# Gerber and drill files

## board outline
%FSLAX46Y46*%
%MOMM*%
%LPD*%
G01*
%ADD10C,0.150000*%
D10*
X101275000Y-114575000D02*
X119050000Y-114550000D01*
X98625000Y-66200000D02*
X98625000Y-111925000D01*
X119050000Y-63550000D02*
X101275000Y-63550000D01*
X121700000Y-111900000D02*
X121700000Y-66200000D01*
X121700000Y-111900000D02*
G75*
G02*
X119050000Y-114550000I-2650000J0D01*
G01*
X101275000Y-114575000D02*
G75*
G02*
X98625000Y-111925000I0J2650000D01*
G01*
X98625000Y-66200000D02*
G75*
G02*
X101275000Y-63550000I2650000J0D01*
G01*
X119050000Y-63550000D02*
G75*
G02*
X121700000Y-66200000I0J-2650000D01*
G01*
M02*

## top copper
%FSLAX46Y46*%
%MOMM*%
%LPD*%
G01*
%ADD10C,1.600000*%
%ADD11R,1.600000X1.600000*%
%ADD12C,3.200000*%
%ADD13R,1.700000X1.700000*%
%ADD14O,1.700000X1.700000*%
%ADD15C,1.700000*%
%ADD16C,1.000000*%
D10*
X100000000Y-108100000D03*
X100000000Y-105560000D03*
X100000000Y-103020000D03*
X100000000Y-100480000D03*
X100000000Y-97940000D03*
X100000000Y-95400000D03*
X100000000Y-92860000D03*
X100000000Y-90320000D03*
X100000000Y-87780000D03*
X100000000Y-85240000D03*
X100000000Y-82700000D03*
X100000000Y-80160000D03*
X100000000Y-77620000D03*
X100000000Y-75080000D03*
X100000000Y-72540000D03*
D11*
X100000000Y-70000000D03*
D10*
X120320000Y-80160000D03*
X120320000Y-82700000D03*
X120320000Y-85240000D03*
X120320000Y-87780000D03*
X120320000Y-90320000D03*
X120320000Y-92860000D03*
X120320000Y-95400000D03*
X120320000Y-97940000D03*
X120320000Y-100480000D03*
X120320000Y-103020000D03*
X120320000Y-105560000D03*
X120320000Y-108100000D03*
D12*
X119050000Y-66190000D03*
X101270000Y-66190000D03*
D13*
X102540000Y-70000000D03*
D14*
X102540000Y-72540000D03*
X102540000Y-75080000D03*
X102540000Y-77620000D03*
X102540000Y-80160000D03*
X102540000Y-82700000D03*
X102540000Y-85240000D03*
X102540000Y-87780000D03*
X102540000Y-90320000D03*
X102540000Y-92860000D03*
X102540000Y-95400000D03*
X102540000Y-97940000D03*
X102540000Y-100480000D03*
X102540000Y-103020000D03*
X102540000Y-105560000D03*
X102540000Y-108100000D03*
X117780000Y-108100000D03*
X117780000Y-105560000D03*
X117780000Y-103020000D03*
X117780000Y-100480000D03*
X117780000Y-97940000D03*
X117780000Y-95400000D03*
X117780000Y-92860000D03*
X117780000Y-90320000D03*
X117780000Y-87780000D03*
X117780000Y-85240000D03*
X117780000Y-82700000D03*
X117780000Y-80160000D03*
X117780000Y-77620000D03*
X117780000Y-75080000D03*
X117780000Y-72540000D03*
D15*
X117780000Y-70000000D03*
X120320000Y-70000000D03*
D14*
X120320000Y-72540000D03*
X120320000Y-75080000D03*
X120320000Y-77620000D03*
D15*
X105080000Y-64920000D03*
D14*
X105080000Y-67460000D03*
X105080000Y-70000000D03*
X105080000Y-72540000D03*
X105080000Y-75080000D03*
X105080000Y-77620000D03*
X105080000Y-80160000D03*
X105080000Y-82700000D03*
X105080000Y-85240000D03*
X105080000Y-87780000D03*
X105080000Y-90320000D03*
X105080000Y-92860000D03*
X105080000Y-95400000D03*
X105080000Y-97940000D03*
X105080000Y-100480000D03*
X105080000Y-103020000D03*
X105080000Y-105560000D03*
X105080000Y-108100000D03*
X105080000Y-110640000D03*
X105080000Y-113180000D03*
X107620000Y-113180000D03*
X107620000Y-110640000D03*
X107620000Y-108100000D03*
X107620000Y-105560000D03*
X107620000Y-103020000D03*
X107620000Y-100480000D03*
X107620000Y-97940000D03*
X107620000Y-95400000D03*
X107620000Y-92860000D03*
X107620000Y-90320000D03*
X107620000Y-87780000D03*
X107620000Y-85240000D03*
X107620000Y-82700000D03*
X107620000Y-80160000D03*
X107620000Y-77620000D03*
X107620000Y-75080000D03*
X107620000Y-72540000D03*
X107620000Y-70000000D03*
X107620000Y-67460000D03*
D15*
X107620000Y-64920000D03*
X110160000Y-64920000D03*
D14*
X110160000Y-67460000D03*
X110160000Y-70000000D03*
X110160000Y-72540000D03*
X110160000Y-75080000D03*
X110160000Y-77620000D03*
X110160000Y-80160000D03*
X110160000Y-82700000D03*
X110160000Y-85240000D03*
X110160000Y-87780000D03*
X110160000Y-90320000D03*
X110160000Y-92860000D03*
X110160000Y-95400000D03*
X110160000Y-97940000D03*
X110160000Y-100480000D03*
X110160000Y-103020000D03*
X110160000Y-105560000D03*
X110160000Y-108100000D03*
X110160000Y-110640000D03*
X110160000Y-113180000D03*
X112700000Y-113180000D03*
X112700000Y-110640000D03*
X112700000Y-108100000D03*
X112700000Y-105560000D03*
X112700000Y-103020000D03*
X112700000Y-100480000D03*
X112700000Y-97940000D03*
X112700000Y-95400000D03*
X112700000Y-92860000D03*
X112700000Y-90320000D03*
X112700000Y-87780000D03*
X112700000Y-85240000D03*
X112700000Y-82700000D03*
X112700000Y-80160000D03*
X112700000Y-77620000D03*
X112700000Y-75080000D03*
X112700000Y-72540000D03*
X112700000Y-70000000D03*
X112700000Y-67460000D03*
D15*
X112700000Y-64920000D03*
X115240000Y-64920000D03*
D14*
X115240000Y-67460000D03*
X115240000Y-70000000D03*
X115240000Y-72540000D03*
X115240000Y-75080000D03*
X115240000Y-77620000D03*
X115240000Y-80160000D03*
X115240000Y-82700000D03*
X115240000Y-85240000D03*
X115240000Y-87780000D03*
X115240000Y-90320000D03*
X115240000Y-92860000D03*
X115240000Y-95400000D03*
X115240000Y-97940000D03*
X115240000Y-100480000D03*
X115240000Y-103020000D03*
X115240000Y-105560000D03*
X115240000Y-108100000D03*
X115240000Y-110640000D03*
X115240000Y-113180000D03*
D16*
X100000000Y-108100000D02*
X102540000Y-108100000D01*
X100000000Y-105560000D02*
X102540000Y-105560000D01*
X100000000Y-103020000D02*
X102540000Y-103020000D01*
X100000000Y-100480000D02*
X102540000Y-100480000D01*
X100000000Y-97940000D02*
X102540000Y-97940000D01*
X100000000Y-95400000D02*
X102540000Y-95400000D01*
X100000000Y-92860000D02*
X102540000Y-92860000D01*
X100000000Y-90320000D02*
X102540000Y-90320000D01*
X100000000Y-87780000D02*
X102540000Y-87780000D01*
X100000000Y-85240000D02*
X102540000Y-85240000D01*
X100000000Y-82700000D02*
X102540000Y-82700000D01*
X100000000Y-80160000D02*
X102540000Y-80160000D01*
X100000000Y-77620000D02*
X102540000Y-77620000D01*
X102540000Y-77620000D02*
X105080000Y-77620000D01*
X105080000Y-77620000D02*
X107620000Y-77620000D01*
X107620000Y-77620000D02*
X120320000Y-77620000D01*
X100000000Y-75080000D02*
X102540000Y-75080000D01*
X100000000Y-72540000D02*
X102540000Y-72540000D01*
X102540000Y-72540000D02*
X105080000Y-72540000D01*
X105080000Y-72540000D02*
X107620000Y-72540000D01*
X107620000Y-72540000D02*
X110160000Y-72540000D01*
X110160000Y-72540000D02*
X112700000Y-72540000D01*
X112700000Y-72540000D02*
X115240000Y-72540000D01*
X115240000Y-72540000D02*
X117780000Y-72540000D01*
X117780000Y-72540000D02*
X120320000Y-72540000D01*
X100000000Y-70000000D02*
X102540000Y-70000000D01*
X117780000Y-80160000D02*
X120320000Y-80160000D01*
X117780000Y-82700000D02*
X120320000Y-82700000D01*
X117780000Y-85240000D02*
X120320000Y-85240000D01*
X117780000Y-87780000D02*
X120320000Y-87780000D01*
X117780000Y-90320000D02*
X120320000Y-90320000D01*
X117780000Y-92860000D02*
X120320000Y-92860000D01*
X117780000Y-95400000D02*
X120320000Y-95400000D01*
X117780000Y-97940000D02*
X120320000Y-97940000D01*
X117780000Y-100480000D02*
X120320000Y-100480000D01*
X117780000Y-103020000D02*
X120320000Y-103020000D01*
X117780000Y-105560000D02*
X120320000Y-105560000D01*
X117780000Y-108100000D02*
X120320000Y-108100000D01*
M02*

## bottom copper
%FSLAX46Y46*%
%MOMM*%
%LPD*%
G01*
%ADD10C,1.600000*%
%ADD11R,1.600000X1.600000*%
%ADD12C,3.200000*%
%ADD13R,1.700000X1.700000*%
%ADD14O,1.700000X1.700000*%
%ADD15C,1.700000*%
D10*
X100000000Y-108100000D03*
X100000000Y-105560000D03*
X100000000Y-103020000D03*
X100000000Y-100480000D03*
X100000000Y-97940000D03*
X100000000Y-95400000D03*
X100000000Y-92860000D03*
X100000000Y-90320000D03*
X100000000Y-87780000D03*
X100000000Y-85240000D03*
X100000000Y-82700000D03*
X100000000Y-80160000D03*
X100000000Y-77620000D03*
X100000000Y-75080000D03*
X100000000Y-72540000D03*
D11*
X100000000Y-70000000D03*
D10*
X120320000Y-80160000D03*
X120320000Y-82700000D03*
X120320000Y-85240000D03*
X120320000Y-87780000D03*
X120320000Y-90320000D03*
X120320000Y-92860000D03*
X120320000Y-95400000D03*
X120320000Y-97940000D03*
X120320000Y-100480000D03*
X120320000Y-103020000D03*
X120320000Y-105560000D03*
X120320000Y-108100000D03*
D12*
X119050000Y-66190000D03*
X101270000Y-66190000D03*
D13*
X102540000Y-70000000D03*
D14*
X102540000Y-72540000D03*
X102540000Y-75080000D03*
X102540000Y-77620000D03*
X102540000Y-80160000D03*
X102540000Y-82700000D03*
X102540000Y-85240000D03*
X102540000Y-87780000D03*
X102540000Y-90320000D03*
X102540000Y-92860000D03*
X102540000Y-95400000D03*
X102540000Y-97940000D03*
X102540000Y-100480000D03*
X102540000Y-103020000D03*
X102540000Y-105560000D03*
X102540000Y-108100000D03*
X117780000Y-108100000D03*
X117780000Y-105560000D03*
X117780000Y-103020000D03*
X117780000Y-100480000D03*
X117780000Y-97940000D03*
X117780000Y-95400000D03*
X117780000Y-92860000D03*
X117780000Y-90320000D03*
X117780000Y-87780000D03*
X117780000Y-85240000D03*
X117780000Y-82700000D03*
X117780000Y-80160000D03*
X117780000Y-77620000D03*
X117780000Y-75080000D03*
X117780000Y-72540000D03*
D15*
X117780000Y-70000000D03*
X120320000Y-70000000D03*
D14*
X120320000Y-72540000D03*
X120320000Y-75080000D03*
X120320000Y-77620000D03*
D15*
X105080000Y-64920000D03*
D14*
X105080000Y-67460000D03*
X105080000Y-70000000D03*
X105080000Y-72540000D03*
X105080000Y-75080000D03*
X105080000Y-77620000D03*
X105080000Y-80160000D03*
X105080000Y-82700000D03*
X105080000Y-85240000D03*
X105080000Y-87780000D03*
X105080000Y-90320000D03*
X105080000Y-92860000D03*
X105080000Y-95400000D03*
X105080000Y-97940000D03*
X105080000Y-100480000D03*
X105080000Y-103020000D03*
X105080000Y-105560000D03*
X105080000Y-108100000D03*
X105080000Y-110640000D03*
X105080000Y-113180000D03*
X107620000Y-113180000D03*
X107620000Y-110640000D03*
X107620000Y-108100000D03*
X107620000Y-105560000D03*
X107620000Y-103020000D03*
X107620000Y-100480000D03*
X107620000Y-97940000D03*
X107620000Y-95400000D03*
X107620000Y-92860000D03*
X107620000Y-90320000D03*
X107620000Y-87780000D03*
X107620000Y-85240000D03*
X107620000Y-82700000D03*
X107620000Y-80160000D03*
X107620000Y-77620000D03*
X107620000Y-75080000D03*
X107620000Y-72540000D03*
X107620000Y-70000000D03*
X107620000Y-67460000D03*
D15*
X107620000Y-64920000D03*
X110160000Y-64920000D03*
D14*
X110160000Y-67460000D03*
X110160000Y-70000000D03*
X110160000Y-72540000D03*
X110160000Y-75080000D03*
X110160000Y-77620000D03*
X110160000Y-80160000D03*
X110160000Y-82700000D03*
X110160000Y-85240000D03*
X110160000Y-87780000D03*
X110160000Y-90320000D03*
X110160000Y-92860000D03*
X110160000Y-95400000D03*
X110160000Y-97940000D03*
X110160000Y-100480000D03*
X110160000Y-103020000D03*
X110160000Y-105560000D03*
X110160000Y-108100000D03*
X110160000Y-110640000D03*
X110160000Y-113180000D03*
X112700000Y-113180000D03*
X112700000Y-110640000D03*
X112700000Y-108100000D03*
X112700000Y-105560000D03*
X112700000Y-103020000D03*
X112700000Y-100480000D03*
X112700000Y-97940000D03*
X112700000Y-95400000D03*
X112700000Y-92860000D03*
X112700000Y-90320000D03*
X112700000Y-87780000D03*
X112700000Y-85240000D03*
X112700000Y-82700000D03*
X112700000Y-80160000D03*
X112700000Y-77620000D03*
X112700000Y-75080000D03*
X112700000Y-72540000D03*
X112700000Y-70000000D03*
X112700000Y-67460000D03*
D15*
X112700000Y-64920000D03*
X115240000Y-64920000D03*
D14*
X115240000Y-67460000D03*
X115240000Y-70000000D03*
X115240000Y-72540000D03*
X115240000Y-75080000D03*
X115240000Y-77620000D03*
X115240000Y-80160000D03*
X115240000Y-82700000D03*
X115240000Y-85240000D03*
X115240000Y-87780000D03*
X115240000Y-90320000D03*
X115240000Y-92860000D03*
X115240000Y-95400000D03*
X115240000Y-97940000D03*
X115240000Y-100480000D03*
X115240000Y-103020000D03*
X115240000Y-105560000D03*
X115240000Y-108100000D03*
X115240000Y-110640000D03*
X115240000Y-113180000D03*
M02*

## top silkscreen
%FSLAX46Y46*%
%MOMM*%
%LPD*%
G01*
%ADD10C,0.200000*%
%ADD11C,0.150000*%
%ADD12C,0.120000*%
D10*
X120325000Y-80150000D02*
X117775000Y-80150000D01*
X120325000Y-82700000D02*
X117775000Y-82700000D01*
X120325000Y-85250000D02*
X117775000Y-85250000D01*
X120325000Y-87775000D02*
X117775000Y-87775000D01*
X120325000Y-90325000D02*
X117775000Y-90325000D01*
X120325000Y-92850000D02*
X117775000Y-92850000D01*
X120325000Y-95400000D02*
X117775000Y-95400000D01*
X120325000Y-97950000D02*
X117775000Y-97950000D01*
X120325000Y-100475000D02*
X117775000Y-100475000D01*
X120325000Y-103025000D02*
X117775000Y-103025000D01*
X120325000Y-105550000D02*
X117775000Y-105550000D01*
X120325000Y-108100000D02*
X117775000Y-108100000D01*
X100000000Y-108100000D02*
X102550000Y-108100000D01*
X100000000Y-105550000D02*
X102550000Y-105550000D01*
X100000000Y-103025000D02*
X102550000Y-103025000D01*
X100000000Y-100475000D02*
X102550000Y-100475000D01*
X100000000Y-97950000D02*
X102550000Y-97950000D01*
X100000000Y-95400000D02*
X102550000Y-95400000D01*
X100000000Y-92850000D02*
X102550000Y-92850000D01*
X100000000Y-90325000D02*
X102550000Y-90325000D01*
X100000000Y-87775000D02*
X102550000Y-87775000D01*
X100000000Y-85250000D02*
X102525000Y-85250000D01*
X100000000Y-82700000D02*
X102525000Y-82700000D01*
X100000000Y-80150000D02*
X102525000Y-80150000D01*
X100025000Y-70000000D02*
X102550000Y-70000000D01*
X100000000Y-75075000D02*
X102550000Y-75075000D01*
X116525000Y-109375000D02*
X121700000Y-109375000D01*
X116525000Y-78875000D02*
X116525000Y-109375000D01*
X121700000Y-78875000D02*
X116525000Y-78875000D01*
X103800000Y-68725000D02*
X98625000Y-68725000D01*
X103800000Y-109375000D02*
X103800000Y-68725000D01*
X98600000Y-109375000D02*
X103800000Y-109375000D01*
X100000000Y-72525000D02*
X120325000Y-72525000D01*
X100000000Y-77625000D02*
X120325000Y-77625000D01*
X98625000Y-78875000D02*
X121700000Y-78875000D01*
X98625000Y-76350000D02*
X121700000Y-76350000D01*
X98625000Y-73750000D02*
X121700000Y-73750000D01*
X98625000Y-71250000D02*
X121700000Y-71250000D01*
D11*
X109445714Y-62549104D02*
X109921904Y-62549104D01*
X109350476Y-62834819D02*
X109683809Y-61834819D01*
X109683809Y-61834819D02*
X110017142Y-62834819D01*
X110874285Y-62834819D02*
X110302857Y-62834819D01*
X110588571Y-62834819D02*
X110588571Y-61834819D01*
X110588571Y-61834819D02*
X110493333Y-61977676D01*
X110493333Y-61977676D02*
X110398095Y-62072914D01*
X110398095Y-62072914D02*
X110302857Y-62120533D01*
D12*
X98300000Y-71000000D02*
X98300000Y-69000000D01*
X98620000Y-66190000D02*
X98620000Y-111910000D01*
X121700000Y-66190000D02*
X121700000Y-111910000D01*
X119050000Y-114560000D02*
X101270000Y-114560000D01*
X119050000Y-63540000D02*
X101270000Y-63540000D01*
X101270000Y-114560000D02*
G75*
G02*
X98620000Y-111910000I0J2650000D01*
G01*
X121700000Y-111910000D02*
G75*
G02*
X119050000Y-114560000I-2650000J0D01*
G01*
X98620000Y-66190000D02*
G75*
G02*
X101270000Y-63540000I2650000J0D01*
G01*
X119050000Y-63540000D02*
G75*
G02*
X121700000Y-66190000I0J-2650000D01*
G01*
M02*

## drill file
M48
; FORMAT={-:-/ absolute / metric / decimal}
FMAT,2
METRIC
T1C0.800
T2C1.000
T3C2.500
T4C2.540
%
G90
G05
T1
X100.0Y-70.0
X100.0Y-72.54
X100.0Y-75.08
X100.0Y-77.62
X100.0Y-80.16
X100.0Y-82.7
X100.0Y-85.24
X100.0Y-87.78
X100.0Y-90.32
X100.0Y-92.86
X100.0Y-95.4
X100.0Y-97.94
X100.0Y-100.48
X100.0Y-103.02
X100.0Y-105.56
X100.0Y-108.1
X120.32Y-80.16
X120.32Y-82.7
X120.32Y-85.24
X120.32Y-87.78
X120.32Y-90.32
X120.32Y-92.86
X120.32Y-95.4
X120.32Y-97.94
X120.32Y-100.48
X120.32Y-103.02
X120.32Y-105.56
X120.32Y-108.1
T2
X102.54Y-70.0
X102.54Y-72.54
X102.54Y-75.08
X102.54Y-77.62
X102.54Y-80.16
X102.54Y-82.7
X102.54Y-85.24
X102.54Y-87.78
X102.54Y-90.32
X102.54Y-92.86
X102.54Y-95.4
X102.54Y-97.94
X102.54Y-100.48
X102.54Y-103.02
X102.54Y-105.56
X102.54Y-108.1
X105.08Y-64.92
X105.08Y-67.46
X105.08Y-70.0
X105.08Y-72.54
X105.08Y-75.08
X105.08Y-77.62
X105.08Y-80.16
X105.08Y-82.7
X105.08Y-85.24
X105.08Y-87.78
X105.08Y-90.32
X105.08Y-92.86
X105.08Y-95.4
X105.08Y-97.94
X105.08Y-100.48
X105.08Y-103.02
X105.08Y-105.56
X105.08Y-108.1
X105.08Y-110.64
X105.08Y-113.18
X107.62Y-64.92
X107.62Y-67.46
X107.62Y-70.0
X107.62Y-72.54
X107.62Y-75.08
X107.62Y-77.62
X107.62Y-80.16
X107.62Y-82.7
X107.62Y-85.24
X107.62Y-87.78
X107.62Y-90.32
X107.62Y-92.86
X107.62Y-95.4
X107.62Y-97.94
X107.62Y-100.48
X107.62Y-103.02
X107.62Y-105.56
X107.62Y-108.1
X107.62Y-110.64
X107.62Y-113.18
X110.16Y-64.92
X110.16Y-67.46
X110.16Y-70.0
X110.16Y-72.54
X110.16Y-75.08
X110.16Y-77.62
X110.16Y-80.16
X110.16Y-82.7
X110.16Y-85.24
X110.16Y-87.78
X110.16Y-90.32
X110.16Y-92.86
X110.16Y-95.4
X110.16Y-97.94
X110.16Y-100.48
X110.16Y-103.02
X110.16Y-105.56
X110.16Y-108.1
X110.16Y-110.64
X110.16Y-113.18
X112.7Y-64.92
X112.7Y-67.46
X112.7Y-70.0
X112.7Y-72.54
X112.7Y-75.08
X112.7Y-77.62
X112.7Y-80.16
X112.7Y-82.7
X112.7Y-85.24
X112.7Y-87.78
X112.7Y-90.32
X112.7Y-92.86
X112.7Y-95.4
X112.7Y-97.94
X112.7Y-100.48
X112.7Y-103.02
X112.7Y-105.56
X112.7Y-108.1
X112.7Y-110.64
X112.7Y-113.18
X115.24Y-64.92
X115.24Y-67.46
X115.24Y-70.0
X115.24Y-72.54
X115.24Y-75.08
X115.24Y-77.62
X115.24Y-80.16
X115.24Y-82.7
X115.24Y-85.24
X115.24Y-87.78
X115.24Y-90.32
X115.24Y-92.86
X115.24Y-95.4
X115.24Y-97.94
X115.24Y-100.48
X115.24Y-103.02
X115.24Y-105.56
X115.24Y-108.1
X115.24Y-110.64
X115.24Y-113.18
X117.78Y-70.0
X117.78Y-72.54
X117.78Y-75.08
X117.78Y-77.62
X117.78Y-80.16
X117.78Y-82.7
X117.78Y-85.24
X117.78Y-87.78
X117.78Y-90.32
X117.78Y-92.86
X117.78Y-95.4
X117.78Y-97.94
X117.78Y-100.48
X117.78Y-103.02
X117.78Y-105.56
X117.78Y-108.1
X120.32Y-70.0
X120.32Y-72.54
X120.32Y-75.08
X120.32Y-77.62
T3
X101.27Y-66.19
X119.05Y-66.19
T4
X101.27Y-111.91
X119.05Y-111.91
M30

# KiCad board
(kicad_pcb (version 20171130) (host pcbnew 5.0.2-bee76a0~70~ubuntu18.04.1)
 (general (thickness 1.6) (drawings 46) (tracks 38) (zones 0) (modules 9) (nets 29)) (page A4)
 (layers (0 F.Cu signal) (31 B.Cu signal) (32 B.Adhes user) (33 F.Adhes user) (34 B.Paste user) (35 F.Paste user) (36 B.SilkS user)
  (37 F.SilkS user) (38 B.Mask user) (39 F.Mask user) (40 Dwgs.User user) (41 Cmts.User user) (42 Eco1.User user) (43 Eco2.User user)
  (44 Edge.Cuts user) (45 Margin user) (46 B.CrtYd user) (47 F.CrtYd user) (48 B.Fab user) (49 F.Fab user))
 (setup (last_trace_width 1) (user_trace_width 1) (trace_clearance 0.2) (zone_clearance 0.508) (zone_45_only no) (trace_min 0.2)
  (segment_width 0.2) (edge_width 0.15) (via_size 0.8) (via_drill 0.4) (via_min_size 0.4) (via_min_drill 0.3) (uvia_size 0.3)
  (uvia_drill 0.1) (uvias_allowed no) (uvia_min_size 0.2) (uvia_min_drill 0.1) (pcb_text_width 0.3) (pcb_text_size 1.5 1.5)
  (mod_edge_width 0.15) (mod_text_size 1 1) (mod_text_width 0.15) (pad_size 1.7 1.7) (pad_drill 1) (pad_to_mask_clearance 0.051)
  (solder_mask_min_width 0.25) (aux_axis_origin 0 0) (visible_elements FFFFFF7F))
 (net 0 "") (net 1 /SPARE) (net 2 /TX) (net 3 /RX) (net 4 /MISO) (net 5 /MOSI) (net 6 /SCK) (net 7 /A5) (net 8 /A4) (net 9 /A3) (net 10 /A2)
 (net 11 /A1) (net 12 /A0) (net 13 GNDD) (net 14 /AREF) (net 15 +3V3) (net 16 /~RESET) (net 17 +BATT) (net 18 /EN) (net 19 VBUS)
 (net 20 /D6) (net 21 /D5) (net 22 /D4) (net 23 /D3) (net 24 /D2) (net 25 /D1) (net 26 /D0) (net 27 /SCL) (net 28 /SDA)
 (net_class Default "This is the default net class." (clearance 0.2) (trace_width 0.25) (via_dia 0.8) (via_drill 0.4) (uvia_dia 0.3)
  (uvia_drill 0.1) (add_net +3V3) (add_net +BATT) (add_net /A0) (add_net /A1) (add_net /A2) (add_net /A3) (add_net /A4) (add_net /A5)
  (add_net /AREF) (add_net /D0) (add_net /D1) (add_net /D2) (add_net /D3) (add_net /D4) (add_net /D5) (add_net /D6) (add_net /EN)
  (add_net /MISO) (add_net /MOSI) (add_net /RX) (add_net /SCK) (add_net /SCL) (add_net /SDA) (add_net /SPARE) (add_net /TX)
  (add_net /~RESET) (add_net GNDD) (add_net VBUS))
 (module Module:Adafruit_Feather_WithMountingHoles (layer F.Cu) (at 100 70)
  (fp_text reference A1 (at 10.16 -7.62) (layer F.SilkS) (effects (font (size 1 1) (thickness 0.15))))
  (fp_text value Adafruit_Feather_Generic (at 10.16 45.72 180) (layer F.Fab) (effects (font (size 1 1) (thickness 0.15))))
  (fp_line (start -1.7 1) (end -1.7 -1) (layer F.SilkS) (width 0.12))
  (fp_line (start -1.38 -3.81) (end -1.38 41.91) (layer F.SilkS) (width 0.12))
  (fp_line (start 21.7 -3.81) (end 21.7 41.91) (layer F.SilkS) (width 0.12))
  (fp_line (start 19.05 44.56) (end 1.27 44.56) (layer F.SilkS) (width 0.12))
  (fp_line (start 19.05 -6.46) (end 1.27 -6.46) (layer F.SilkS) (width 0.12))
  (fp_arc (start 1.27 41.91) (end -1.38 41.91) (angle -90) (layer F.SilkS) (width 0.12))
  (fp_arc (start 19.05 41.91) (end 19.05 44.56) (angle -90) (layer F.SilkS) (width 0.12))
  (fp_arc (start 1.27 -3.81) (end 1.27 -6.46) (angle -90) (layer F.SilkS) (width 0.12))
  (fp_arc (start 19.05 -3.81) (end 21.7 -3.81) (angle -90) (layer F.SilkS) (width 0.12))
  (pad 16 thru_hole circle (at 0 38.1 180) (size 1.6 1.6) (drill 0.8) (layers *.Cu *.Mask) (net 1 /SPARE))
  (pad 15 thru_hole circle (at 0 35.56 180) (size 1.6 1.6) (drill 0.8) (layers *.Cu *.Mask) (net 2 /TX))
  (pad 14 thru_hole circle (at 0 33.02 180) (size 1.6 1.6) (drill 0.8) (layers *.Cu *.Mask) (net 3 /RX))
  (pad 13 thru_hole circle (at 0 30.48 180) (size 1.6 1.6) (drill 0.8) (layers *.Cu *.Mask) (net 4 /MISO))
  (pad 12 thru_hole circle (at 0 27.94 180) (size 1.6 1.6) (drill 0.8) (layers *.Cu *.Mask) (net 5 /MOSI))
  (pad 11 thru_hole circle (at 0 25.4 180) (size 1.6 1.6) (drill 0.8) (layers *.Cu *.Mask) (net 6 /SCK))
  (pad 10 thru_hole circle (at 0 22.86 180) (size 1.6 1.6) (drill 0.8) (layers *.Cu *.Mask) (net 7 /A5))
  (pad 9 thru_hole circle (at 0 20.32 180) (size 1.6 1.6) (drill 0.8) (layers *.Cu *.Mask) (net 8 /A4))
  (pad 8 thru_hole circle (at 0 17.78 180) (size 1.6 1.6) (drill 0.8) (layers *.Cu *.Mask) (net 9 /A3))
  (pad 7 thru_hole circle (at 0 15.24 180) (size 1.6 1.6) (drill 0.8) (layers *.Cu *.Mask) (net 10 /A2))
  (pad 6 thru_hole circle (at 0 12.7 180) (size 1.6 1.6) (drill 0.8) (layers *.Cu *.Mask) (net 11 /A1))
  (pad 5 thru_hole circle (at 0 10.16 180) (size 1.6 1.6) (drill 0.8) (layers *.Cu *.Mask) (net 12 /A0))
  (pad 4 thru_hole circle (at 0 7.62 180) (size 1.6 1.6) (drill 0.8) (layers *.Cu *.Mask) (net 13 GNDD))
  (pad 3 thru_hole circle (at 0 5.08 180) (size 1.6 1.6) (drill 0.8) (layers *.Cu *.Mask) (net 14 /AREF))
  (pad 2 thru_hole circle (at 0 2.54 180) (size 1.6 1.6) (drill 0.8) (layers *.Cu *.Mask) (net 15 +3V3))
  (pad 1 thru_hole rect (at 0 0 180) (size 1.6 1.6) (drill 0.8) (layers *.Cu *.Mask) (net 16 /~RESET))
  (pad 28 thru_hole circle (at 20.32 10.16 180) (size 1.6 1.6) (drill 0.8) (layers *.Cu *.Mask) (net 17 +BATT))
  (pad 27 thru_hole circle (at 20.32 12.7 180) (size 1.6 1.6) (drill 0.8) (layers *.Cu *.Mask) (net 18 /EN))
  (pad 26 thru_hole circle (at 20.32 15.24 180) (size 1.6 1.6) (drill 0.8) (layers *.Cu *.Mask) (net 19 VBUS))
  (pad 25 thru_hole circle (at 20.32 17.78 180) (size 1.6 1.6) (drill 0.8) (layers *.Cu *.Mask) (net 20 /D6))
  (pad 24 thru_hole circle (at 20.32 20.32 180) (size 1.6 1.6) (drill 0.8) (layers *.Cu *.Mask) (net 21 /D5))
  (pad 23 thru_hole circle (at 20.32 22.86 180) (size 1.6 1.6) (drill 0.8) (layers *.Cu *.Mask) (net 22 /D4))
  (pad 22 thru_hole circle (at 20.32 25.4 180) (size 1.6 1.6) (drill 0.8) (layers *.Cu *.Mask) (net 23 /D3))
  (pad 21 thru_hole circle (at 20.32 27.94 180) (size 1.6 1.6) (drill 0.8) (layers *.Cu *.Mask) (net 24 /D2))
  (pad 20 thru_hole circle (at 20.32 30.48 180) (size 1.6 1.6) (drill 0.8) (layers *.Cu *.Mask) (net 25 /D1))
  (pad 19 thru_hole circle (at 20.32 33.02 180) (size 1.6 1.6) (drill 0.8) (layers *.Cu *.Mask) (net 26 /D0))
  (pad 18 thru_hole circle (at 20.32 35.56 180) (size 1.6 1.6) (drill 0.8) (layers *.Cu *.Mask) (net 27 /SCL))
  (pad 17 thru_hole circle (at 20.32 38.1 180) (size 1.6 1.6) (drill 0.8) (layers *.Cu *.Mask) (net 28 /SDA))
  (pad "" np_thru_hole circle (at 19.05 -3.81 270) (size 3.2 3.2) (drill 2.5) (layers *.Cu *.Mask))
  (pad "" np_thru_hole circle (at 19.05 41.91 270) (size 2.54 2.54) (drill 2.54) (layers *.Cu *.Mask))
  (pad "" np_thru_hole circle (at 1.27 -3.81 270) (size 3.2 3.2) (drill 2.5) (layers *.Cu *.Mask))
  (pad "" np_thru_hole circle (at 1.27 41.91 270) (size 2.54 2.54) (drill 2.54) (layers *.Cu *.Mask)))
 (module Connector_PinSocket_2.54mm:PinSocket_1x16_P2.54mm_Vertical (layer B.Cu) (at 102.54 70 180)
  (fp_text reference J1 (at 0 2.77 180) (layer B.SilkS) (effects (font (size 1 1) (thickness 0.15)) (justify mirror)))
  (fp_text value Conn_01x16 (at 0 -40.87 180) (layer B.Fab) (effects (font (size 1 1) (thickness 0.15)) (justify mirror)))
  (pad 1 thru_hole rect (at 0 0 180) (size 1.7 1.7) (drill 1) (layers *.Cu *.Mask) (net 16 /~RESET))
  (pad 2 thru_hole oval (at 0 -2.54 180) (size 1.7 1.7) (drill 1) (layers *.Cu *.Mask) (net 15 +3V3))
  (pad 3 thru_hole oval (at 0 -5.08 180) (size 1.7 1.7) (drill 1) (layers *.Cu *.Mask) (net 14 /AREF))
  (pad 4 thru_hole oval (at 0 -7.62 180) (size 1.7 1.7) (drill 1) (layers *.Cu *.Mask) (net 13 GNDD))
  (pad 5 thru_hole oval (at 0 -10.16 180) (size 1.7 1.7) (drill 1) (layers *.Cu *.Mask) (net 12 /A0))
  (pad 6 thru_hole oval (at 0 -12.7 180) (size 1.7 1.7) (drill 1) (layers *.Cu *.Mask) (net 11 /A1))
  (pad 7 thru_hole oval (at 0 -15.24 180) (size 1.7 1.7) (drill 1) (layers *.Cu *.Mask) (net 10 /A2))
  (pad 8 thru_hole oval (at 0 -17.78 180) (size 1.7 1.7) (drill 1) (layers *.Cu *.Mask) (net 9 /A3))
  (pad 9 thru_hole oval (at 0 -20.32 180) (size 1.7 1.7) (drill 1) (layers *.Cu *.Mask) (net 8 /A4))
  (pad 10 thru_hole oval (at 0 -22.86 180) (size 1.7 1.7) (drill 1) (layers *.Cu *.Mask) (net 7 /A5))
  (pad 11 thru_hole oval (at 0 -25.4 180) (size 1.7 1.7) (drill 1) (layers *.Cu *.Mask) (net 6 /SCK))
  (pad 12 thru_hole oval (at 0 -27.94 180) (size 1.7 1.7) (drill 1) (layers *.Cu *.Mask) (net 5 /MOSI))
  (pad 13 thru_hole oval (at 0 -30.48 180) (size 1.7 1.7) (drill 1) (layers *.Cu *.Mask) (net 4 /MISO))
  (pad 14 thru_hole oval (at 0 -33.02 180) (size 1.7 1.7) (drill 1) (layers *.Cu *.Mask) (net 3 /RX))
  (pad 15 thru_hole oval (at 0 -35.56 180) (size 1.7 1.7) (drill 1) (layers *.Cu *.Mask) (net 2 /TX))
  (pad 16 thru_hole oval (at 0 -38.1 180) (size 1.7 1.7) (drill 1) (layers *.Cu *.Mask) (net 1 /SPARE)))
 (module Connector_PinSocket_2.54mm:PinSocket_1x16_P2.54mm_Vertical (layer B.Cu) (at 117.78 70 180)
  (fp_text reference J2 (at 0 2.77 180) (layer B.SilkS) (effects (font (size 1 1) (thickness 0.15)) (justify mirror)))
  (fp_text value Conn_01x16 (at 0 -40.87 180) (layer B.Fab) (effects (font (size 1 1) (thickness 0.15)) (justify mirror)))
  (pad 16 thru_hole oval (at 0 -38.1 180) (size 1.7 1.7) (drill 1) (layers *.Cu *.Mask) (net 28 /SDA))
  (pad 15 thru_hole oval (at 0 -35.56 180) (size 1.7 1.7) (drill 1) (layers *.Cu *.Mask) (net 27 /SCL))
  (pad 14 thru_hole oval (at 0 -33.02 180) (size 1.7 1.7) (drill 1) (layers *.Cu *.Mask) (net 26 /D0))
  (pad 13 thru_hole oval (at 0 -30.48 180) (size 1.7 1.7) (drill 1) (layers *.Cu *.Mask) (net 25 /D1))
  (pad 12 thru_hole oval (at 0 -27.94 180) (size 1.7 1.7) (drill 1) (layers *.Cu *.Mask) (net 24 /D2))
  (pad 11 thru_hole oval (at 0 -25.4 180) (size 1.7 1.7) (drill 1) (layers *.Cu *.Mask) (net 23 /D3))
  (pad 10 thru_hole oval (at 0 -22.86 180) (size 1.7 1.7) (drill 1) (layers *.Cu *.Mask) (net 22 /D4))
  (pad 9 thru_hole oval (at 0 -20.32 180) (size 1.7 1.7) (drill 1) (layers *.Cu *.Mask) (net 21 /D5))
  (pad 8 thru_hole oval (at 0 -17.78 180) (size 1.7 1.7) (drill 1) (layers *.Cu *.Mask) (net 20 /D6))
  (pad 7 thru_hole oval (at 0 -15.24 180) (size 1.7 1.7) (drill 1) (layers *.Cu *.Mask) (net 19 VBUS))
  (pad 6 thru_hole oval (at 0 -12.7 180) (size 1.7 1.7) (drill 1) (layers *.Cu *.Mask) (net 18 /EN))
  (pad 5 thru_hole oval (at 0 -10.16 180) (size 1.7 1.7) (drill 1) (layers *.Cu *.Mask) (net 17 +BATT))
  (pad 4 thru_hole oval (at 0 -7.62 180) (size 1.7 1.7) (drill 1) (layers *.Cu *.Mask) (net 13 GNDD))
  (pad 3 thru_hole oval (at 0 -5.08 180) (size 1.7 1.7) (drill 1) (layers *.Cu *.Mask))
  (pad 2 thru_hole oval (at 0 -2.54 180) (size 1.7 1.7) (drill 1) (layers *.Cu *.Mask) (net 15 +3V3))
  (pad 1 thru_hole circle (at 0 0 180) (size 1.7 1.7) (drill 1) (layers *.Cu *.Mask)))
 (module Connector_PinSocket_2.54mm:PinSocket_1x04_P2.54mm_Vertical (layer B.Cu) (at 120.32 70 180)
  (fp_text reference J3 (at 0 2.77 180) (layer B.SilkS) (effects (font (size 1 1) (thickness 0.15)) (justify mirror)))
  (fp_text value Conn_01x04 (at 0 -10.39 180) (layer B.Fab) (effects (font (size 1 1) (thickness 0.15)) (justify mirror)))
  (pad 1 thru_hole circle (at 0 0 180) (size 1.7 1.7) (drill 1) (layers *.Cu *.Mask))
  (pad 2 thru_hole oval (at 0 -2.54 180) (size 1.7 1.7) (drill 1) (layers *.Cu *.Mask) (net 15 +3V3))
  (pad 3 thru_hole oval (at 0 -5.08 180) (size 1.7 1.7) (drill 1) (layers *.Cu *.Mask))
  (pad 4 thru_hole oval (at 0 -7.62 180) (size 1.7 1.7) (drill 1) (layers *.Cu *.Mask) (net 13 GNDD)))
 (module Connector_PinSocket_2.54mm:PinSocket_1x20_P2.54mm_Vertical (layer B.Cu) (at 105.08 64.92 180)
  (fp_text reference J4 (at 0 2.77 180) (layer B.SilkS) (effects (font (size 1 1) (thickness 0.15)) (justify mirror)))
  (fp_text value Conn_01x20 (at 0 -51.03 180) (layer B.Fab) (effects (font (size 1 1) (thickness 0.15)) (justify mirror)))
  (pad 1 thru_hole circle (at 0 0 180) (size 1.7 1.7) (drill 1) (layers *.Cu *.Mask))
  (pad 2 thru_hole oval (at 0 -2.54 180) (size 1.7 1.7) (drill 1) (layers *.Cu *.Mask))
  (pad 3 thru_hole oval (at 0 -5.08 180) (size 1.7 1.7) (drill 1) (layers *.Cu *.Mask))
  (pad 4 thru_hole oval (at 0 -7.62 180) (size 1.7 1.7) (drill 1) (layers *.Cu *.Mask) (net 15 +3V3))
  (pad 5 thru_hole oval (at 0 -10.16 180) (size 1.7 1.7) (drill 1) (layers *.Cu *.Mask))
  (pad 6 thru_hole oval (at 0 -12.7 180) (size 1.7 1.7) (drill 1) (layers *.Cu *.Mask) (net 13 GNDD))
  (pad 7 thru_hole oval (at 0 -15.24 180) (size 1.7 1.7) (drill 1) (layers *.Cu *.Mask))
  (pad 8 thru_hole oval (at 0 -17.78 180) (size 1.7 1.7) (drill 1) (layers *.Cu *.Mask))
  (pad 9 thru_hole oval (at 0 -20.32 180) (size 1.7 1.7) (drill 1) (layers *.Cu *.Mask))
  (pad 10 thru_hole oval (at 0 -22.86 180) (size 1.7 1.7) (drill 1) (layers *.Cu *.Mask))
  (pad 11 thru_hole oval (at 0 -25.4 180) (size 1.7 1.7) (drill 1) (layers *.Cu *.Mask))
  (pad 12 thru_hole oval (at 0 -27.94 180) (size 1.7 1.7) (drill 1) (layers *.Cu *.Mask))
  (pad 13 thru_hole oval (at 0 -30.48 180) (size 1.7 1.7) (drill 1) (layers *.Cu *.Mask))
  (pad 14 thru_hole oval (at 0 -33.02 180) (size 1.7 1.7) (drill 1) (layers *.Cu *.Mask))
  (pad 15 thru_hole oval (at 0 -35.56 180) (size 1.7 1.7) (drill 1) (layers *.Cu *.Mask))
  (pad 16 thru_hole oval (at 0 -38.1 180) (size 1.7 1.7) (drill 1) (layers *.Cu *.Mask))
  (pad 17 thru_hole oval (at 0 -40.64 180) (size 1.7 1.7) (drill 1) (layers *.Cu *.Mask))
  (pad 18 thru_hole oval (at 0 -43.18 180) (size 1.7 1.7) (drill 1) (layers *.Cu *.Mask))
  (pad 19 thru_hole oval (at 0 -45.72 180) (size 1.7 1.7) (drill 1) (layers *.Cu *.Mask))
  (pad 20 thru_hole oval (at 0 -48.26 180) (size 1.7 1.7) (drill 1) (layers *.Cu *.Mask)))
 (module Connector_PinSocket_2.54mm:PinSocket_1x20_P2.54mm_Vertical (layer B.Cu) (at 107.62 64.92 180)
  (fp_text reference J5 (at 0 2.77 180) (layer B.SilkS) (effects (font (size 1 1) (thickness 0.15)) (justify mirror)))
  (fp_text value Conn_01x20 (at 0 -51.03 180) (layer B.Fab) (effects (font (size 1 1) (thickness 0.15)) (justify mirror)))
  (pad 20 thru_hole oval (at 0 -48.26 180) (size 1.7 1.7) (drill 1) (layers *.Cu *.Mask))
  (pad 19 thru_hole oval (at 0 -45.72 180) (size 1.7 1.7) (drill 1) (layers *.Cu *.Mask))
  (pad 18 thru_hole oval (at 0 -43.18 180) (size 1.7 1.7) (drill 1) (layers *.Cu *.Mask))
  (pad 17 thru_hole oval (at 0 -40.64 180) (size 1.7 1.7) (drill 1) (layers *.Cu *.Mask))
  (pad 16 thru_hole oval (at 0 -38.1 180) (size 1.7 1.7) (drill 1) (layers *.Cu *.Mask))
  (pad 15 thru_hole oval (at 0 -35.56 180) (size 1.7 1.7) (drill 1) (layers *.Cu *.Mask))
  (pad 14 thru_hole oval (at 0 -33.02 180) (size 1.7 1.7) (drill 1) (layers *.Cu *.Mask))
  (pad 13 thru_hole oval (at 0 -30.48 180) (size 1.7 1.7) (drill 1) (layers *.Cu *.Mask))
  (pad 12 thru_hole oval (at 0 -27.94 180) (size 1.7 1.7) (drill 1) (layers *.Cu *.Mask))
  (pad 11 thru_hole oval (at 0 -25.4 180) (size 1.7 1.7) (drill 1) (layers *.Cu *.Mask))
  (pad 10 thru_hole oval (at 0 -22.86 180) (size 1.7 1.7) (drill 1) (layers *.Cu *.Mask))
  (pad 9 thru_hole oval (at 0 -20.32 180) (size 1.7 1.7) (drill 1) (layers *.Cu *.Mask))
  (pad 8 thru_hole oval (at 0 -17.78 180) (size 1.7 1.7) (drill 1) (layers *.Cu *.Mask))
  (pad 7 thru_hole oval (at 0 -15.24 180) (size 1.7 1.7) (drill 1) (layers *.Cu *.Mask))
  (pad 6 thru_hole oval (at 0 -12.7 180) (size 1.7 1.7) (drill 1) (layers *.Cu *.Mask) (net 13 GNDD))
  (pad 5 thru_hole oval (at 0 -10.16 180) (size 1.7 1.7) (drill 1) (layers *.Cu *.Mask))
  (pad 4 thru_hole oval (at 0 -7.62 180) (size 1.7 1.7) (drill 1) (layers *.Cu *.Mask) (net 15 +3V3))
  (pad 3 thru_hole oval (at 0 -5.08 180) (size 1.7 1.7) (drill 1) (layers *.Cu *.Mask))
  (pad 2 thru_hole oval (at 0 -2.54 180) (size 1.7 1.7) (drill 1) (layers *.Cu *.Mask))
  (pad 1 thru_hole circle (at 0 0 180) (size 1.7 1.7) (drill 1) (layers *.Cu *.Mask)))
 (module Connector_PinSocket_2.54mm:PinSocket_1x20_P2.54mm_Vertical (layer B.Cu) (at 110.16 64.92 180)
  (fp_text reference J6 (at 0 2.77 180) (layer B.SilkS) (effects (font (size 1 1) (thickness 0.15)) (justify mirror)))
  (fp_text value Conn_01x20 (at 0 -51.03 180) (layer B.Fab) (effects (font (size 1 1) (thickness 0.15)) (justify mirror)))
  (pad 1 thru_hole circle (at 0 0 180) (size 1.7 1.7) (drill 1) (layers *.Cu *.Mask))
  (pad 2 thru_hole oval (at 0 -2.54 180) (size 1.7 1.7) (drill 1) (layers *.Cu *.Mask))
  (pad 3 thru_hole oval (at 0 -5.08 180) (size 1.7 1.7) (drill 1) (layers *.Cu *.Mask))
  (pad 4 thru_hole oval (at 0 -7.62 180) (size 1.7 1.7) (drill 1) (layers *.Cu *.Mask) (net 15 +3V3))
  (pad 5 thru_hole oval (at 0 -10.16 180) (size 1.7 1.7) (drill 1) (layers *.Cu *.Mask))
  (pad 6 thru_hole oval (at 0 -12.7 180) (size 1.7 1.7) (drill 1) (layers *.Cu *.Mask) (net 13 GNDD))
  (pad 7 thru_hole oval (at 0 -15.24 180) (size 1.7 1.7) (drill 1) (layers *.Cu *.Mask))
  (pad 8 thru_hole oval (at 0 -17.78 180) (size 1.7 1.7) (drill 1) (layers *.Cu *.Mask))
  (pad 9 thru_hole oval (at 0 -20.32 180) (size 1.7 1.7) (drill 1) (layers *.Cu *.Mask))
  (pad 10 thru_hole oval (at 0 -22.86 180) (size 1.7 1.7) (drill 1) (layers *.Cu *.Mask))
  (pad 11 thru_hole oval (at 0 -25.4 180) (size 1.7 1.7) (drill 1) (layers *.Cu *.Mask))
  (pad 12 thru_hole oval (at 0 -27.94 180) (size 1.7 1.7) (drill 1) (layers *.Cu *.Mask))
  (pad 13 thru_hole oval (at 0 -30.48 180) (size 1.7 1.7) (drill 1) (layers *.Cu *.Mask))
  (pad 14 thru_hole oval (at 0 -33.02 180) (size 1.7 1.7) (drill 1) (layers *.Cu *.Mask))
  (pad 15 thru_hole oval (at 0 -35.56 180) (size 1.7 1.7) (drill 1) (layers *.Cu *.Mask))
  (pad 16 thru_hole oval (at 0 -38.1 180) (size 1.7 1.7) (drill 1) (layers *.Cu *.Mask))
  (pad 17 thru_hole oval (at 0 -40.64 180) (size 1.7 1.7) (drill 1) (layers *.Cu *.Mask))
  (pad 18 thru_hole oval (at 0 -43.18 180) (size 1.7 1.7) (drill 1) (layers *.Cu *.Mask))
  (pad 19 thru_hole oval (at 0 -45.72 180) (size 1.7 1.7) (drill 1) (layers *.Cu *.Mask))
  (pad 20 thru_hole oval (at 0 -48.26 180) (size 1.7 1.7) (drill 1) (layers *.Cu *.Mask)))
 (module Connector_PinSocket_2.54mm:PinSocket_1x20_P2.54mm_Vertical (layer B.Cu) (at 112.7 64.92 180)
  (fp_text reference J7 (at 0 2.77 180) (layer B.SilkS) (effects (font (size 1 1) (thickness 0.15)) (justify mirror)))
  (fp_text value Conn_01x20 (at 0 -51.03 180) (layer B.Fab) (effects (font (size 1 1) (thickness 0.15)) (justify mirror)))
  (pad 20 thru_hole oval (at 0 -48.26 180) (size 1.7 1.7) (drill 1) (layers *.Cu *.Mask))
  (pad 19 thru_hole oval (at 0 -45.72 180) (size 1.7 1.7) (drill 1) (layers *.Cu *.Mask))
  (pad 18 thru_hole oval (at 0 -43.18 180) (size 1.7 1.7) (drill 1) (layers *.Cu *.Mask))
  (pad 17 thru_hole oval (at 0 -40.64 180) (size 1.7 1.7) (drill 1) (layers *.Cu *.Mask))
  (pad 16 thru_hole oval (at 0 -38.1 180) (size 1.7 1.7) (drill 1) (layers *.Cu *.Mask))
  (pad 15 thru_hole oval (at 0 -35.56 180) (size 1.7 1.7) (drill 1) (layers *.Cu *.Mask))
  (pad 14 thru_hole oval (at 0 -33.02 180) (size 1.7 1.7) (drill 1) (layers *.Cu *.Mask))
  (pad 13 thru_hole oval (at 0 -30.48 180) (size 1.7 1.7) (drill 1) (layers *.Cu *.Mask))
  (pad 12 thru_hole oval (at 0 -27.94 180) (size 1.7 1.7) (drill 1) (layers *.Cu *.Mask))
  (pad 11 thru_hole oval (at 0 -25.4 180) (size 1.7 1.7) (drill 1) (layers *.Cu *.Mask))
  (pad 10 thru_hole oval (at 0 -22.86 180) (size 1.7 1.7) (drill 1) (layers *.Cu *.Mask))
  (pad 9 thru_hole oval (at 0 -20.32 180) (size 1.7 1.7) (drill 1) (layers *.Cu *.Mask))
  (pad 8 thru_hole oval (at 0 -17.78 180) (size 1.7 1.7) (drill 1) (layers *.Cu *.Mask))
  (pad 7 thru_hole oval (at 0 -15.24 180) (size 1.7 1.7) (drill 1) (layers *.Cu *.Mask))
  (pad 6 thru_hole oval (at 0 -12.7 180) (size 1.7 1.7) (drill 1) (layers *.Cu *.Mask) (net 13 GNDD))
  (pad 5 thru_hole oval (at 0 -10.16 180) (size 1.7 1.7) (drill 1) (layers *.Cu *.Mask))
  (pad 4 thru_hole oval (at 0 -7.62 180) (size 1.7 1.7) (drill 1) (layers *.Cu *.Mask) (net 15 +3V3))
  (pad 3 thru_hole oval (at 0 -5.08 180) (size 1.7 1.7) (drill 1) (layers *.Cu *.Mask))
  (pad 2 thru_hole oval (at 0 -2.54 180) (size 1.7 1.7) (drill 1) (layers *.Cu *.Mask))
  (pad 1 thru_hole circle (at 0 0 180) (size 1.7 1.7) (drill 1) (layers *.Cu *.Mask)))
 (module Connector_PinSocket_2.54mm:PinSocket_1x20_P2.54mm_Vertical (layer B.Cu) (at 115.24 64.92 180)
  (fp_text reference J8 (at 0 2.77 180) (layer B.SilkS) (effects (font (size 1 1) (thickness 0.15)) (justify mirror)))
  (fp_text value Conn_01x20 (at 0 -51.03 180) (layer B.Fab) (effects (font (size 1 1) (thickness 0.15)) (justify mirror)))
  (pad 1 thru_hole circle (at 0 0 180) (size 1.7 1.7) (drill 1) (layers *.Cu *.Mask))
  (pad 2 thru_hole oval (at 0 -2.54 180) (size 1.7 1.7) (drill 1) (layers *.Cu *.Mask))
  (pad 3 thru_hole oval (at 0 -5.08 180) (size 1.7 1.7) (drill 1) (layers *.Cu *.Mask))
  (pad 4 thru_hole oval (at 0 -7.62 180) (size 1.7 1.7) (drill 1) (layers *.Cu *.Mask) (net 15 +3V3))
  (pad 5 thru_hole oval (at 0 -10.16 180) (size 1.7 1.7) (drill 1) (layers *.Cu *.Mask))
  (pad 6 thru_hole oval (at 0 -12.7 180) (size 1.7 1.7) (drill 1) (layers *.Cu *.Mask) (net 13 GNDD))
  (pad 7 thru_hole oval (at 0 -15.24 180) (size 1.7 1.7) (drill 1) (layers *.Cu *.Mask))
  (pad 8 thru_hole oval (at 0 -17.78 180) (size 1.7 1.7) (drill 1) (layers *.Cu *.Mask))
  (pad 9 thru_hole oval (at 0 -20.32 180) (size 1.7 1.7) (drill 1) (layers *.Cu *.Mask))
  (pad 10 thru_hole oval (at 0 -22.86 180) (size 1.7 1.7) (drill 1) (layers *.Cu *.Mask))
  (pad 11 thru_hole oval (at 0 -25.4 180) (size 1.7 1.7) (drill 1) (layers *.Cu *.Mask))
  (pad 12 thru_hole oval (at 0 -27.94 180) (size 1.7 1.7) (drill 1) (layers *.Cu *.Mask))
  (pad 13 thru_hole oval (at 0 -30.48 180) (size 1.7 1.7) (drill 1) (layers *.Cu *.Mask))
  (pad 14 thru_hole oval (at 0 -33.02 180) (size 1.7 1.7) (drill 1) (layers *.Cu *.Mask))
  (pad 15 thru_hole oval (at 0 -35.56 180) (size 1.7 1.7) (drill 1) (layers *.Cu *.Mask))
  (pad 16 thru_hole oval (at 0 -38.1 180) (size 1.7 1.7) (drill 1) (layers *.Cu *.Mask))
  (pad 17 thru_hole oval (at 0 -40.64 180) (size 1.7 1.7) (drill 1) (layers *.Cu *.Mask))
  (pad 18 thru_hole oval (at 0 -43.18 180) (size 1.7 1.7) (drill 1) (layers *.Cu *.Mask))
  (pad 19 thru_hole oval (at 0 -45.72 180) (size 1.7 1.7) (drill 1) (layers *.Cu *.Mask))
  (pad 20 thru_hole oval (at 0 -48.26 180) (size 1.7 1.7) (drill 1) (layers *.Cu *.Mask)))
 (gr_line (start 120.325 80.15) (end 117.775 80.15) (layer F.SilkS) (width 0.2))
 (gr_line (start 120.325 82.7) (end 117.775 82.7) (layer F.SilkS) (width 0.2))
 (gr_line (start 120.325 85.25) (end 117.775 85.25) (layer F.SilkS) (width 0.2))
 (gr_line (start 120.325 87.775) (end 117.775 87.775) (layer F.SilkS) (width 0.2))
 (gr_line (start 120.325 90.325) (end 117.775 90.325) (layer F.SilkS) (width 0.2))
 (gr_line (start 120.325 92.85) (end 117.775 92.85) (layer F.SilkS) (width 0.2))
 (gr_line (start 120.325 95.4) (end 117.775 95.4) (layer F.SilkS) (width 0.2))
 (gr_line (start 120.325 97.95) (end 117.775 97.95) (layer F.SilkS) (width 0.2))
 (gr_line (start 120.325 100.475) (end 117.775 100.475) (layer F.SilkS) (width 0.2))
 (gr_line (start 120.325 103.025) (end 117.775 103.025) (layer F.SilkS) (width 0.2))
 (gr_line (start 120.325 105.55) (end 117.775 105.55) (layer F.SilkS) (width 0.2))
 (gr_line (start 120.325 108.1) (end 117.775 108.1) (layer F.SilkS) (width 0.2))
 (gr_line (start 100 108.1) (end 102.55 108.1) (layer F.SilkS) (width 0.2))
 (gr_line (start 100 105.55) (end 102.55 105.55) (layer F.SilkS) (width 0.2))
 (gr_line (start 100 103.025) (end 102.55 103.025) (layer F.SilkS) (width 0.2))
 (gr_line (start 100 100.475) (end 102.55 100.475) (layer F.SilkS) (width 0.2))
 (gr_line (start 100 97.95) (end 102.55 97.95) (layer F.SilkS) (width 0.2))
 (gr_line (start 100 95.4) (end 102.55 95.4) (layer F.SilkS) (width 0.2))
 (gr_line (start 100 92.85) (end 102.55 92.85) (layer F.SilkS) (width 0.2))
 (gr_line (start 100 90.325) (end 102.55 90.325) (layer F.SilkS) (width 0.2))
 (gr_line (start 100 87.775) (end 102.55 87.775) (layer F.SilkS) (width 0.2))
 (gr_line (start 100 85.25) (end 102.525 85.25) (layer F.SilkS) (width 0.2))
 (gr_line (start 100 82.7) (end 102.525 82.7) (layer F.SilkS) (width 0.2))
 (gr_line (start 100 80.15) (end 102.525 80.15) (layer F.SilkS) (width 0.2))
 (gr_line (start 100.025 70) (end 102.55 70) (layer F.SilkS) (width 0.2))
 (gr_line (start 100 75.075) (end 102.55 75.075) (layer F.SilkS) (width 0.2))
 (gr_line (start 116.525 109.375) (end 121.7 109.375) (layer F.SilkS) (width 0.2))
 (gr_line (start 116.525 78.875) (end 116.525 109.375) (layer F.SilkS) (width 0.2))
 (gr_line (start 121.7 78.875) (end 116.525 78.875) (layer F.SilkS) (width 0.2))
 (gr_line (start 103.8 68.725) (end 98.625 68.725) (layer F.SilkS) (width 0.2))
 (gr_line (start 103.8 109.375) (end 103.8 68.725) (layer F.SilkS) (width 0.2))
 (gr_line (start 98.6 109.375) (end 103.8 109.375) (layer F.SilkS) (width 0.2))
 (gr_line (start 100 72.525) (end 120.325 72.525) (layer F.SilkS) (width 0.2))
 (gr_line (start 100 77.625) (end 120.325 77.625) (layer F.SilkS) (width 0.2))
 (gr_line (start 98.625 78.875) (end 121.7 78.875) (layer F.SilkS) (width 0.2))
 (gr_line (start 98.625 76.35) (end 121.7 76.35) (layer F.SilkS) (width 0.2))
 (gr_line (start 98.625 73.75) (end 121.7 73.75) (layer F.SilkS) (width 0.2))
 (gr_line (start 98.625 71.25) (end 121.7 71.25) (layer F.SilkS) (width 0.2))
 (gr_line (start 101.275 114.575) (end 119.05 114.55) (layer Edge.Cuts) (width 0.15))
 (gr_line (start 98.625 66.2) (end 98.625 111.925) (layer Edge.Cuts) (width 0.15))
 (gr_line (start 119.05 63.55) (end 101.275 63.55) (layer Edge.Cuts) (width 0.15))
 (gr_line (start 121.7 111.9) (end 121.7 66.2) (layer Edge.Cuts) (width 0.15))
 (gr_arc (start 119.05 111.9) (end 119.05 114.55) (angle -90) (layer Edge.Cuts) (width 0.15))
 (gr_arc (start 101.275 111.925) (end 98.625 111.925) (angle -90) (layer Edge.Cuts) (width 0.15))
 (gr_arc (start 101.275 66.2) (end 101.275 63.55) (angle -90) (layer Edge.Cuts) (width 0.15))
 (gr_arc (start 119.05 66.2) (end 121.7 66.2) (angle -90) (layer Edge.Cuts) (width 0.15))
 (segment (start 100 108.1) (end 102.54 108.1) (width 1) (layer F.Cu) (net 1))
 (segment (start 100 105.56) (end 102.54 105.56) (width 1) (layer F.Cu) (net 2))
 (segment (start 100 103.02) (end 102.54 103.02) (width 1) (layer F.Cu) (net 3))
 (segment (start 100 100.48) (end 102.54 100.48) (width 1) (layer F.Cu) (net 4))
 (segment (start 100 97.94) (end 102.54 97.94) (width 1) (layer F.Cu) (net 5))
 (segment (start 100 95.4) (end 102.54 95.4) (width 1) (layer F.Cu) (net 6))
 (segment (start 100 92.86) (end 102.54 92.86) (width 1) (layer F.Cu) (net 7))
 (segment (start 100 90.32) (end 102.54 90.32) (width 1) (layer F.Cu) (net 8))
 (segment (start 100 87.78) (end 102.54 87.78) (width 1) (layer F.Cu) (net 9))
 (segment (start 100 85.24) (end 102.54 85.24) (width 1) (layer F.Cu) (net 10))
 (segment (start 100 82.7) (end 102.54 82.7) (width 1) (layer F.Cu) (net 11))
 (segment (start 100 80.16) (end 102.54 80.16) (width 1) (layer F.Cu) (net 12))
 (segment (start 100 77.62) (end 102.54 77.62) (width 1) (layer F.Cu) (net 13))
 (segment (start 102.54 77.62) (end 105.08 77.62) (width 1) (layer F.Cu) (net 13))
 (segment (start 105.08 77.62) (end 107.62 77.62) (width 1) (layer F.Cu) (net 13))
 (segment (start 107.62 77.62) (end 120.32 77.62) (width 1) (layer F.Cu) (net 13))
 (segment (start 100 75.08) (end 102.54 75.08) (width 1) (layer F.Cu) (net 14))
 (segment (start 100 72.54) (end 102.54 72.54) (width 1) (layer F.Cu) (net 15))
 (segment (start 102.54 72.54) (end 105.08 72.54) (width 1) (layer F.Cu) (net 15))
 (segment (start 105.08 72.54) (end 107.62 72.54) (width 1) (layer F.Cu) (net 15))
 (segment (start 107.62 72.54) (end 110.16 72.54) (width 1) (layer F.Cu) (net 15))
 (segment (start 110.16 72.54) (end 112.7 72.54) (width 1) (layer F.Cu) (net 15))
 (segment (start 112.7 72.54) (end 115.24 72.54) (width 1) (layer F.Cu) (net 15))
 (segment (start 115.24 72.54) (end 117.78 72.54) (width 1) (layer F.Cu) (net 15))
 (segment (start 117.78 72.54) (end 120.32 72.54) (width 1) (layer F.Cu) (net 15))
 (segment (start 100 70) (end 102.54 70) (width 1) (layer F.Cu) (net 16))
 (segment (start 117.78 80.16) (end 120.32 80.16) (width 1) (layer F.Cu) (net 17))
 (segment (start 117.78 82.7) (end 120.32 82.7) (width 1) (layer F.Cu) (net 18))
 (segment (start 117.78 85.24) (end 120.32 85.24) (width 1) (layer F.Cu) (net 19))
 (segment (start 117.78 87.78) (end 120.32 87.78) (width 1) (layer F.Cu) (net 20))
 (segment (start 117.78 90.32) (end 120.32 90.32) (width 1) (layer F.Cu) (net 21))
 (segment (start 117.78 92.86) (end 120.32 92.86) (width 1) (layer F.Cu) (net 22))
 (segment (start 117.78 95.4) (end 120.32 95.4) (width 1) (layer F.Cu) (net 23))
 (segment (start 117.78 97.94) (end 120.32 97.94) (width 1) (layer F.Cu) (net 24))
 (segment (start 117.78 100.48) (end 120.32 100.48) (width 1) (layer F.Cu) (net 25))
 (segment (start 117.78 103.02) (end 120.32 103.02) (width 1) (layer F.Cu) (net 26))
 (segment (start 117.78 105.56) (end 120.32 105.56) (width 1) (layer F.Cu) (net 27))
 (segment (start 117.78 108.1) (end 120.32 108.1) (width 1) (layer F.Cu) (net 28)))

